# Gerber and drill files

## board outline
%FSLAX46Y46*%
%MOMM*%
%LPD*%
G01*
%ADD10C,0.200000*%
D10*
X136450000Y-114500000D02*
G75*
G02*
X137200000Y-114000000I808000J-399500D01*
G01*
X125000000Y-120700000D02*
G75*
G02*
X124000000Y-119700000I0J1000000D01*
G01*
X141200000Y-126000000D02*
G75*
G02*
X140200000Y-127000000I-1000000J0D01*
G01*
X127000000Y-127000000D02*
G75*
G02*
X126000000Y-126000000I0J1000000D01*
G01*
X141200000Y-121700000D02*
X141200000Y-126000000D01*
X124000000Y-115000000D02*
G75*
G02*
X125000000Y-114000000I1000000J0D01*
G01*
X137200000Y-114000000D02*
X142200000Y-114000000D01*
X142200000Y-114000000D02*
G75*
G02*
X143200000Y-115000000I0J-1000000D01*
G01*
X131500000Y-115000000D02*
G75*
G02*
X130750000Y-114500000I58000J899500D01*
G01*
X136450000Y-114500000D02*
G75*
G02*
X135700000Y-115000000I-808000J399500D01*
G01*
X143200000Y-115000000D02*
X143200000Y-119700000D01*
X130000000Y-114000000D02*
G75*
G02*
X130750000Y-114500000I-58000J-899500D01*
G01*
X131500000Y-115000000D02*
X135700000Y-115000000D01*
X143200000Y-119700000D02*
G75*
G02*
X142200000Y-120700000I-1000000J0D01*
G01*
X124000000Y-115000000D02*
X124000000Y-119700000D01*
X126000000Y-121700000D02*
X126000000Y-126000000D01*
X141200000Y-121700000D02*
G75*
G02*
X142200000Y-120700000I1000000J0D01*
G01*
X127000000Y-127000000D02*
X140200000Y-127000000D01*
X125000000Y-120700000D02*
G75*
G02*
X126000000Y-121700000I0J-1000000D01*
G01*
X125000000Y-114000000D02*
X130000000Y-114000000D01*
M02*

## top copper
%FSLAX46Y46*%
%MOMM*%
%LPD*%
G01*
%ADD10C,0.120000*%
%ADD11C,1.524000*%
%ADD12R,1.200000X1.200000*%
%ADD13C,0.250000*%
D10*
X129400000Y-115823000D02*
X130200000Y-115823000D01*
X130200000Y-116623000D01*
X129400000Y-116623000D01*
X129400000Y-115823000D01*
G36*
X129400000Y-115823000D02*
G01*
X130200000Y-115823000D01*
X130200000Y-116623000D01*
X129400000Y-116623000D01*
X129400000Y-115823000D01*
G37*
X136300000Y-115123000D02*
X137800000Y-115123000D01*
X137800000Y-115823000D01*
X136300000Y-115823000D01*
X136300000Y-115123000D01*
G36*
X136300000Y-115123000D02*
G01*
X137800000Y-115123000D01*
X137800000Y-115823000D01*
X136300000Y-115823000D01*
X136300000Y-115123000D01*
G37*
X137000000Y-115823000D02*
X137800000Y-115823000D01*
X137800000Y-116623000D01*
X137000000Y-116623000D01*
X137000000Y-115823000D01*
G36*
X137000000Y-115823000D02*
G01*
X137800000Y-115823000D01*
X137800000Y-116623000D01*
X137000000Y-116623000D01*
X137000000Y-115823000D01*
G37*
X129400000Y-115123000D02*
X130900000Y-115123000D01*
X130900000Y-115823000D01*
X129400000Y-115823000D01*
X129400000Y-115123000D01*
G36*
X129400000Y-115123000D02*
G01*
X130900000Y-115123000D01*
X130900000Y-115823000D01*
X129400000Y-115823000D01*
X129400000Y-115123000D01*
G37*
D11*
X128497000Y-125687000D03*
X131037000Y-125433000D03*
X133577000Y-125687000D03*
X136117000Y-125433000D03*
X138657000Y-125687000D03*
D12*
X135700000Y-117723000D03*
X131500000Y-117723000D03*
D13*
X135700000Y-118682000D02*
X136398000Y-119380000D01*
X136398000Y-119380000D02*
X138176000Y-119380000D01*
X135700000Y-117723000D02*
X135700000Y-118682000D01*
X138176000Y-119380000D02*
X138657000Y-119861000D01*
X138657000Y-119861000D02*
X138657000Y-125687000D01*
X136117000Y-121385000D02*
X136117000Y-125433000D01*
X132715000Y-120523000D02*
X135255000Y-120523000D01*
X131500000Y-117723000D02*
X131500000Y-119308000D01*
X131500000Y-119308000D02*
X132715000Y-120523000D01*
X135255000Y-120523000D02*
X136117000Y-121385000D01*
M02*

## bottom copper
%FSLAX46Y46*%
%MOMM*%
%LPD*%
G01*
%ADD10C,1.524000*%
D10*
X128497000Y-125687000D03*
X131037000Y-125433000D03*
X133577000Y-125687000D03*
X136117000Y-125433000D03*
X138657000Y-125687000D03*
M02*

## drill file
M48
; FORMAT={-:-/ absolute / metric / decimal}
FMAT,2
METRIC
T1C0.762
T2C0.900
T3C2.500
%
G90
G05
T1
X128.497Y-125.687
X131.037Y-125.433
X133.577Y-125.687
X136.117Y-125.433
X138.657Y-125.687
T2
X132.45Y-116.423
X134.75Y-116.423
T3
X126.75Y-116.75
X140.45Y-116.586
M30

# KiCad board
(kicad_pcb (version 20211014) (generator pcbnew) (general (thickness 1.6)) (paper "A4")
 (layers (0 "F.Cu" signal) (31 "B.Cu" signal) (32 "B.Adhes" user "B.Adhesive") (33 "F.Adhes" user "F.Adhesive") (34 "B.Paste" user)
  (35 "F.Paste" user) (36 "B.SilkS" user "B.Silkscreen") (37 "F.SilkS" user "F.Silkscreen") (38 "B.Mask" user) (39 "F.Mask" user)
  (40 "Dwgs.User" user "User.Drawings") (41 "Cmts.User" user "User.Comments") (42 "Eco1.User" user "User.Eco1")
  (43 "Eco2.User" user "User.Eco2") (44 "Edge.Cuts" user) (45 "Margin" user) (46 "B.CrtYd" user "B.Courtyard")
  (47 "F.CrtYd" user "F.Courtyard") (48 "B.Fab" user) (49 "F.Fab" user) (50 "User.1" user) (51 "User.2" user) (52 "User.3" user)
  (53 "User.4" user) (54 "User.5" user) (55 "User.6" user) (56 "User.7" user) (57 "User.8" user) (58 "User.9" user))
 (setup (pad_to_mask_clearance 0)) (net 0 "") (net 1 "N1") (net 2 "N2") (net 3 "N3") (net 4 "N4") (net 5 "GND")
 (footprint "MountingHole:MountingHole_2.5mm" (layer "F.Cu") (at 126.75 116.75)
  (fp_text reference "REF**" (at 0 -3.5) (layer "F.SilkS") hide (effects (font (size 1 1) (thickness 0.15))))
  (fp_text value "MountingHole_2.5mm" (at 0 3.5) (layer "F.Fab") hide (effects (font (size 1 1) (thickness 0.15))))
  (pad "" np_thru_hole circle (at 0 0) (size 2.5 2.5) (drill 2.5) (layers *.Cu *.Mask)))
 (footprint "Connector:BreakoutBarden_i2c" (layer "F.Cu") (at 133.477 120.607)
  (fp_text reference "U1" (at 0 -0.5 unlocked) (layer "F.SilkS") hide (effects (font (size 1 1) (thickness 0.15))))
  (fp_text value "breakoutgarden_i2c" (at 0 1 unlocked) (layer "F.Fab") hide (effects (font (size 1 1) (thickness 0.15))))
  (pad "1" thru_hole circle (at -4.98 5.08) (size 1.524 1.524) (drill 0.762) (layers *.Cu *.Mask) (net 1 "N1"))
  (pad "2" thru_hole circle (at -2.44 4.826) (size 1.524 1.524) (drill 0.762) (layers *.Cu *.Mask) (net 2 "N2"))
  (pad "3" thru_hole circle (at 0.1 5.08) (size 1.524 1.524) (drill 0.762) (layers *.Cu *.Mask) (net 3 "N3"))
  (pad "4" thru_hole circle (at 2.64 4.826) (size 1.524 1.524) (drill 0.762) (layers *.Cu *.Mask) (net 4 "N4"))
  (pad "5" thru_hole circle (at 5.18 5.08) (size 1.524 1.524) (drill 0.762) (layers *.Cu *.Mask) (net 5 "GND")))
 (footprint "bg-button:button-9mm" (layer "F.Cu") (at 133.477 119.634)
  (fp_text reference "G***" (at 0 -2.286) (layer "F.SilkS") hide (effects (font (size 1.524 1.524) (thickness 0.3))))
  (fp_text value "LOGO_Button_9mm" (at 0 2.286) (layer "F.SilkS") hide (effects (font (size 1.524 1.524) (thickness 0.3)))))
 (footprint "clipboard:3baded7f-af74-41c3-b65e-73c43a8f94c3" (layer "F.Cu") (at 147.955 120.396)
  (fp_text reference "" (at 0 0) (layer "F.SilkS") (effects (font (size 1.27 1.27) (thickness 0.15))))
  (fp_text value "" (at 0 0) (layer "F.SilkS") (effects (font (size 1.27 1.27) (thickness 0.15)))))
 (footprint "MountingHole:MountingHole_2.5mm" (layer "F.Cu") (at 140.45 116.586)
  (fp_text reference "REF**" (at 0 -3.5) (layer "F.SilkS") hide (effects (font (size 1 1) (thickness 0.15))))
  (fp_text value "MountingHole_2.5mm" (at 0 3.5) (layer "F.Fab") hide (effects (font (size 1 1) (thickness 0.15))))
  (pad "" np_thru_hole circle (at 0 0) (size 2.5 2.5) (drill 2.5) (layers *.Cu *.Mask)))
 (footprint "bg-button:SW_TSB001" (layer "F.Cu") (at 129.4 115.123)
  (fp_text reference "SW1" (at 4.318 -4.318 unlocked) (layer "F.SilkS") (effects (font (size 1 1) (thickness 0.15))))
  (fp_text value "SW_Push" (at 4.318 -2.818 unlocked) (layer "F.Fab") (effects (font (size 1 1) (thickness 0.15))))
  (fp_rect (start 0 0.7) (end 0.8 1.5) (layer "F.Cu") (width 0.12) (fill solid))
  (fp_rect (start 6.9 0) (end 8.4 0.7) (layer "F.Cu") (width 0.12) (fill solid))
  (fp_rect (start 7.6 0.7) (end 8.4 1.5) (layer "F.Cu") (width 0.12) (fill solid))
  (fp_rect (start 0 0) (end 1.5 0.7) (layer "F.Cu") (width 0.12) (fill solid))
  (pad "" np_thru_hole circle (at 3.05 1.3) (size 0.9 0.9) (drill 0.9) (layers F&B.Cu *.Mask))
  (pad "" np_thru_hole circle (at 5.35 1.3) (size 0.9 0.9) (drill 0.9) (layers F&B.Cu *.Mask))
  (pad "1" smd rect (at 6.3 2.6) (size 1.2 1.2) (layers "F.Cu" "F.Paste" "F.Mask") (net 5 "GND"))
  (pad "2" smd rect (at 2.1 2.6) (size 1.2 1.2) (layers "F.Cu" "F.Paste" "F.Mask") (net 4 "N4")))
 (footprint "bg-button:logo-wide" (layer "B.Cu") (at 133.604 118.872 180)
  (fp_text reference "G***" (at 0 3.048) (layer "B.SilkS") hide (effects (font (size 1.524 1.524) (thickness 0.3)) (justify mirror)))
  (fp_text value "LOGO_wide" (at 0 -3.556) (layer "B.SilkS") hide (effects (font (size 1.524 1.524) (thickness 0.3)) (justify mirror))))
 (gr_arc (start 136.45 114.5) (mid 136.758013 114.149519) (end 137.2 114) (layer "Edge.Cuts") (width 0.2))
 (gr_arc (start 125 120.7) (mid 124.292893 120.407107) (end 124 119.7) (layer "Edge.Cuts") (width 0.2))
 (gr_arc (start 141.2 126) (mid 140.907107 126.707107) (end 140.2 127) (layer "Edge.Cuts") (width 0.2))
 (gr_arc (start 127 127) (mid 126.292893 126.707107) (end 126 126) (layer "Edge.Cuts") (width 0.2))
 (gr_line (start 141.2 121.7) (end 141.2 126) (layer "Edge.Cuts") (width 0.2))
 (gr_arc (start 124 115) (mid 124.292893 114.292893) (end 125 114) (layer "Edge.Cuts") (width 0.2))
 (gr_line (start 137.2 114) (end 142.2 114) (layer "Edge.Cuts") (width 0.2))
 (gr_arc (start 142.2 114) (mid 142.907107 114.292893) (end 143.2 115) (layer "Edge.Cuts") (width 0.2))
 (gr_arc (start 131.5 115) (mid 131.058013 114.850481) (end 130.75 114.5) (layer "Edge.Cuts") (width 0.2))
 (gr_arc (start 136.45 114.5) (mid 136.141987 114.850481) (end 135.7 115) (layer "Edge.Cuts") (width 0.2))
 (gr_line (start 143.2 115) (end 143.2 119.7) (layer "Edge.Cuts") (width 0.2))
 (gr_arc (start 130 114) (mid 130.441987 114.149519) (end 130.75 114.5) (layer "Edge.Cuts") (width 0.2))
 (gr_line (start 131.5 115) (end 135.7 115) (layer "Edge.Cuts") (width 0.2))
 (gr_arc (start 143.2 119.7) (mid 142.907107 120.407107) (end 142.2 120.7) (layer "Edge.Cuts") (width 0.2))
 (gr_line (start 124 115) (end 124 119.7) (layer "Edge.Cuts") (width 0.2))
 (gr_line (start 126 121.7) (end 126 126) (layer "Edge.Cuts") (width 0.2))
 (gr_arc (start 141.2 121.7) (mid 141.492893 120.992893) (end 142.2 120.7) (layer "Edge.Cuts") (width 0.2))
 (gr_line (start 127 127) (end 140.2 127) (layer "Edge.Cuts") (width 0.2))
 (gr_arc (start 125 120.7) (mid 125.707107 120.992893) (end 126 121.7) (layer "Edge.Cuts") (width 0.2))
 (gr_line (start 125 114) (end 130 114) (layer "Edge.Cuts") (width 0.2))
 (segment (start 135.7 118.682) (end 136.398 119.38) (width 0.25) (layer "F.Cu") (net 5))
 (segment (start 136.398 119.38) (end 138.176 119.38) (width 0.25) (layer "F.Cu") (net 5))
 (segment (start 135.7 117.723) (end 135.7 118.682) (width 0.25) (layer "F.Cu") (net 5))
 (segment (start 138.176 119.38) (end 138.657 119.861) (width 0.25) (layer "F.Cu") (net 5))
 (segment (start 138.657 119.861) (end 138.657 125.687) (width 0.25) (layer "F.Cu") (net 5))
 (segment (start 136.117 121.385) (end 136.117 125.433) (width 0.25) (layer "F.Cu") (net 4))
 (segment (start 132.715 120.523) (end 135.255 120.523) (width 0.25) (layer "F.Cu") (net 4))
 (segment (start 131.5 117.723) (end 131.5 119.308) (width 0.25) (layer "F.Cu") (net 4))
 (segment (start 131.5 119.308) (end 132.715 120.523) (width 0.25) (layer "F.Cu") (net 4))
 (segment (start 135.255 120.523) (end 136.117 121.385) (width 0.25) (layer "F.Cu") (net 4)))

